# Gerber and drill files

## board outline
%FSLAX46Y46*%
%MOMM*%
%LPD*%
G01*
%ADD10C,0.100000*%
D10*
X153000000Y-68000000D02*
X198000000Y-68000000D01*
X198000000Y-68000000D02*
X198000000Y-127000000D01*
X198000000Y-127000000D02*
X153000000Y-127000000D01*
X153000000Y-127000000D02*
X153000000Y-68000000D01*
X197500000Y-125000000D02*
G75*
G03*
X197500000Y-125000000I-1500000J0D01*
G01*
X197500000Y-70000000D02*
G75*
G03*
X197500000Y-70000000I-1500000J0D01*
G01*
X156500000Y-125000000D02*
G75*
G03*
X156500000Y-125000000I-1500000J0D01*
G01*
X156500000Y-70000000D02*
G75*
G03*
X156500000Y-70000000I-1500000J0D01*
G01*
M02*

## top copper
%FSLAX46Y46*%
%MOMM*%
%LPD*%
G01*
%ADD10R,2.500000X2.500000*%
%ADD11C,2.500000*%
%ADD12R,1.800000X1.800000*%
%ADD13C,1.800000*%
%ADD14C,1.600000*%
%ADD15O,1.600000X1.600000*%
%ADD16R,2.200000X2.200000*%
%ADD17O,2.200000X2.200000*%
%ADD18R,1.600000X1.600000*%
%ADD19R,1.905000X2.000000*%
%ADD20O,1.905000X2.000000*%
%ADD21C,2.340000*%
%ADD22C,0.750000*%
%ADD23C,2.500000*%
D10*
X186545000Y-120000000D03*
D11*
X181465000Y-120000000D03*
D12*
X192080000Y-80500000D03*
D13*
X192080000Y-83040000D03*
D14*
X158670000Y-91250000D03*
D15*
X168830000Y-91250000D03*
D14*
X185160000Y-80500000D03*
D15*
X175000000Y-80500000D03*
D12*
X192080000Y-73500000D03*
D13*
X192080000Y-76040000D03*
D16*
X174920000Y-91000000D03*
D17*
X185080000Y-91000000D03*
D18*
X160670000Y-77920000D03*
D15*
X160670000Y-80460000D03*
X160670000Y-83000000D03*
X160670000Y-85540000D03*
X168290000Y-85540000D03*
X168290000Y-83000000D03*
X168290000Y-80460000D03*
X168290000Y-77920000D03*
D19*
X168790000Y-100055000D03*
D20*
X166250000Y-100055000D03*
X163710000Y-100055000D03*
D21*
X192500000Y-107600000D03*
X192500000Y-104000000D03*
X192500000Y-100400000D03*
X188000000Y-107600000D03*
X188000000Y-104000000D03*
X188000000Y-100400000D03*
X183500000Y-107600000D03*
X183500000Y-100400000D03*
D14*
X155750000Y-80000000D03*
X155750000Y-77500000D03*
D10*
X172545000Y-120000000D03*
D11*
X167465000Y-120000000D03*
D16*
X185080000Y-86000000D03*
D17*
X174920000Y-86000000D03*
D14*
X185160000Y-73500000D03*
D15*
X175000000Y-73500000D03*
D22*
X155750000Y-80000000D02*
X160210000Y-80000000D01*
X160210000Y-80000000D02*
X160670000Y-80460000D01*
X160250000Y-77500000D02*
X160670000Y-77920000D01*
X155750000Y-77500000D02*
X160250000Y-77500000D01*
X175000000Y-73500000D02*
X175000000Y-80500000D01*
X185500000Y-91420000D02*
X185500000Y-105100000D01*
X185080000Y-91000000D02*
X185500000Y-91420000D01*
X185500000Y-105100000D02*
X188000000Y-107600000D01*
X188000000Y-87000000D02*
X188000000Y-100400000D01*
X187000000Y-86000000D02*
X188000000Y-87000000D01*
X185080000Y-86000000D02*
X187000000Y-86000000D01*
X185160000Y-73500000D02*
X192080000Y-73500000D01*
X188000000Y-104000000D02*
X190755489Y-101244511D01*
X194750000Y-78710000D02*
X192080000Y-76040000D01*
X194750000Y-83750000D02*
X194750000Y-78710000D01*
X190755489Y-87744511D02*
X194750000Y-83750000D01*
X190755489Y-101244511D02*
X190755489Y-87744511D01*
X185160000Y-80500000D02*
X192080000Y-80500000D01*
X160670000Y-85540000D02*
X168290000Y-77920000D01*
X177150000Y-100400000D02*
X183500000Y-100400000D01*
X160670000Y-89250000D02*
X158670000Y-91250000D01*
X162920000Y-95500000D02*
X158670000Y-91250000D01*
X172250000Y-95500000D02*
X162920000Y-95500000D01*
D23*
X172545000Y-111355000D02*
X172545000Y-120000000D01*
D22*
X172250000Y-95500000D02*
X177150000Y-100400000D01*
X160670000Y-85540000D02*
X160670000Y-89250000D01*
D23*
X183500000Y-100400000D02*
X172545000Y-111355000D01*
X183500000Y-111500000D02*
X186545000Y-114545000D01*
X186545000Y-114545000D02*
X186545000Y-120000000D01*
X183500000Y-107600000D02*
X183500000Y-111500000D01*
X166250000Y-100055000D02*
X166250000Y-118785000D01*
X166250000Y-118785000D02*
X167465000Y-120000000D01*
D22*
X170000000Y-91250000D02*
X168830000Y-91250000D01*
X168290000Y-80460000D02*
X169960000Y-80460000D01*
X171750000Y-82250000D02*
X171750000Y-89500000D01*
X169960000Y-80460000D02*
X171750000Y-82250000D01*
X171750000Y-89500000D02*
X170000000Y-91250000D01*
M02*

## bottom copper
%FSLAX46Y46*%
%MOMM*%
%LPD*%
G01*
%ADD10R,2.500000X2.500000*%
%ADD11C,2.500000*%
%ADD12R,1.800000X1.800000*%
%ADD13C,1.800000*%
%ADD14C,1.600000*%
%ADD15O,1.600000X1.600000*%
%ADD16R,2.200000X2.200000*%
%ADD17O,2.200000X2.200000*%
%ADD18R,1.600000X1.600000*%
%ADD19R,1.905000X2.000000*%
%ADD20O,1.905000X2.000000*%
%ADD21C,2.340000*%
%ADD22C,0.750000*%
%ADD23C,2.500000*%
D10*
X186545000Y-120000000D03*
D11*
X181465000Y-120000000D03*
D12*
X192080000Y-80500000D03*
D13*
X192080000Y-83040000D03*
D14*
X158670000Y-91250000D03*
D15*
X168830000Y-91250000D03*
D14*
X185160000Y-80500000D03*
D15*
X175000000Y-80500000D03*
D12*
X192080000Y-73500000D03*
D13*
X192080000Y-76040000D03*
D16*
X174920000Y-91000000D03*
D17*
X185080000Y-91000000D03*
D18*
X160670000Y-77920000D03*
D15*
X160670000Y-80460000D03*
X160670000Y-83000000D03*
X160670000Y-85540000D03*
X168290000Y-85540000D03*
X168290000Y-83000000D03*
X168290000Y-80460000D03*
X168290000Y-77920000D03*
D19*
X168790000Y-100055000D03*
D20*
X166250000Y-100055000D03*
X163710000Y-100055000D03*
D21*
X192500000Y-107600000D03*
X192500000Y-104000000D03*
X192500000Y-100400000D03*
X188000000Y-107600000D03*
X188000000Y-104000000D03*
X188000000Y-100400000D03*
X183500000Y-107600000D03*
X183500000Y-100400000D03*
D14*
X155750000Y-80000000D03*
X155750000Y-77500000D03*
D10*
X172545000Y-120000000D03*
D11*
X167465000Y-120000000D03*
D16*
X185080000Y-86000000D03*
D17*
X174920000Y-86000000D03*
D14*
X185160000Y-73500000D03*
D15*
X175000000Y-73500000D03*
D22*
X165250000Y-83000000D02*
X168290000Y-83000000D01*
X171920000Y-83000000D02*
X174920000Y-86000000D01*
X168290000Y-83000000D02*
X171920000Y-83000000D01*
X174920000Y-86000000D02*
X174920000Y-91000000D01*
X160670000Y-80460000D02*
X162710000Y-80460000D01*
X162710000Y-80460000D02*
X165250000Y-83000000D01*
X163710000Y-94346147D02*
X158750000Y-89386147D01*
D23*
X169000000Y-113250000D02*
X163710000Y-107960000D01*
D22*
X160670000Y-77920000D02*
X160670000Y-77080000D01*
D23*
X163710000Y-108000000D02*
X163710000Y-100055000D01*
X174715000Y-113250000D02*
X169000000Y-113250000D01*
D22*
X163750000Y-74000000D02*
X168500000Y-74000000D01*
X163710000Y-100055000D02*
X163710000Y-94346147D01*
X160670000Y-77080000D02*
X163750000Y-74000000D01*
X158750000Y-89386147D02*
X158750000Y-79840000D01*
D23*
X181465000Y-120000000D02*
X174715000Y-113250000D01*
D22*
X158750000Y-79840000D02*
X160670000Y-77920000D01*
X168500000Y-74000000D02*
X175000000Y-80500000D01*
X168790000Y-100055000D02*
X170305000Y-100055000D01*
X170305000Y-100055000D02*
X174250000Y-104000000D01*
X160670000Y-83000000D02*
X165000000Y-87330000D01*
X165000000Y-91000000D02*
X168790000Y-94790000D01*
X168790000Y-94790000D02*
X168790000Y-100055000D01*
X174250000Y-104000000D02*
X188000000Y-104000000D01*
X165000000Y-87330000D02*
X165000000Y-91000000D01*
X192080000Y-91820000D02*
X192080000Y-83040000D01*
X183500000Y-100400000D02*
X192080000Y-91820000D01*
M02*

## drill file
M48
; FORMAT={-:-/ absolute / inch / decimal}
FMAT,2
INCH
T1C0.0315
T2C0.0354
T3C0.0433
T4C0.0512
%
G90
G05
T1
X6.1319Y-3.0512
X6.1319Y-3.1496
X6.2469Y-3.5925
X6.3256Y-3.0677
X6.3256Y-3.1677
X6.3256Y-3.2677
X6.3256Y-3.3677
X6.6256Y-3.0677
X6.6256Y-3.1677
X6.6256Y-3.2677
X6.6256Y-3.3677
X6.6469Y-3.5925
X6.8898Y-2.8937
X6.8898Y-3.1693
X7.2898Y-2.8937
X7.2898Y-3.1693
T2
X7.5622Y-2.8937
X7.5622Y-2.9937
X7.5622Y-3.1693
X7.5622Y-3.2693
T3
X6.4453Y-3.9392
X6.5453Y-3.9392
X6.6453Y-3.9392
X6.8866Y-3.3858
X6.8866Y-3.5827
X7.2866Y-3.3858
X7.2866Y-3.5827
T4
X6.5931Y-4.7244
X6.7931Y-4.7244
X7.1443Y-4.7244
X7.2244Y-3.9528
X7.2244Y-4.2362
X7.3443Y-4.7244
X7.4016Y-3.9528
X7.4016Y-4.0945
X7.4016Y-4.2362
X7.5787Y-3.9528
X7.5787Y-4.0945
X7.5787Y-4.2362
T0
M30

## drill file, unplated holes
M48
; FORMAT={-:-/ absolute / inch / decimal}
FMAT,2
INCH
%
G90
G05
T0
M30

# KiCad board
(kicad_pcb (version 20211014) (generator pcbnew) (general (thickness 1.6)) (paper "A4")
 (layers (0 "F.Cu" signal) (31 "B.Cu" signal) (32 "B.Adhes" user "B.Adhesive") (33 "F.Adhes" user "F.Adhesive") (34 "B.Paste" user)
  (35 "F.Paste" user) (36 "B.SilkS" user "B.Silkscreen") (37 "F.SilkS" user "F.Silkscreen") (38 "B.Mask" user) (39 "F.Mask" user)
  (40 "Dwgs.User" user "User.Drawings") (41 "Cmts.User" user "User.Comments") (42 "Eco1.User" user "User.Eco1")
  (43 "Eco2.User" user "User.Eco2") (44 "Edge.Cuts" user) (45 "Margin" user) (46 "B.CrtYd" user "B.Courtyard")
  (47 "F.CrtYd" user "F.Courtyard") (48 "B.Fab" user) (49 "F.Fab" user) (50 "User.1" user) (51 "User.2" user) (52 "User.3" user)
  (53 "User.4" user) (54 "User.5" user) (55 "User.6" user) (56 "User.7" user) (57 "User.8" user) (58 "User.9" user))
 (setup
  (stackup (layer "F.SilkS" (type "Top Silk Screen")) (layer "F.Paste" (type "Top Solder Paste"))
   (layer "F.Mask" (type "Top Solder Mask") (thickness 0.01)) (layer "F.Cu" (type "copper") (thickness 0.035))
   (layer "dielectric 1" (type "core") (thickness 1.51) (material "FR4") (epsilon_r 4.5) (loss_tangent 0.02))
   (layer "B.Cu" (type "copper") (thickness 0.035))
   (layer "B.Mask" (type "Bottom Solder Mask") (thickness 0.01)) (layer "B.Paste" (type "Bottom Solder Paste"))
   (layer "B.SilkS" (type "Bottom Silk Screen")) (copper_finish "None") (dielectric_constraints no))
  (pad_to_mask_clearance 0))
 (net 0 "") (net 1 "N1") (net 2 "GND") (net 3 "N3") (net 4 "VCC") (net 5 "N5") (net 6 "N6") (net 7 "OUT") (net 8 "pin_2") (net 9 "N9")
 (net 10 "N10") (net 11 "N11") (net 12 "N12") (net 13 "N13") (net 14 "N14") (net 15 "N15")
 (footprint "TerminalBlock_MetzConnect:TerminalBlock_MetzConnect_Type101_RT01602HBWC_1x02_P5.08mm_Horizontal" (layer "F.Cu")
  (at 186.545 120 180)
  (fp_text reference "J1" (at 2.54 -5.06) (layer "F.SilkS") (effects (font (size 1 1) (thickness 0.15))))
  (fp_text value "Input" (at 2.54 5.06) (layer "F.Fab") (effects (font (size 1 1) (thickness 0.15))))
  (pad "1" thru_hole rect (at 0 0 180) (size 2.5 2.5) (drill 1.3) (layers *.Cu *.Mask) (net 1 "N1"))
  (pad "2" thru_hole circle (at 5.08 0 180) (size 2.5 2.5) (drill 1.3) (layers *.Cu *.Mask) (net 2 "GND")))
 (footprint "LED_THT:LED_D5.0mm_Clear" (layer "F.Cu") (at 192.08 80.5 -90)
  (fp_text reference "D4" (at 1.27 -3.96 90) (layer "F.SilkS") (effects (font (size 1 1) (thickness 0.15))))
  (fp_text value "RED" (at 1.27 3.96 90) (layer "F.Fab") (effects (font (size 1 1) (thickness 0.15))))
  (pad "1" thru_hole rect (at 0 0 270) (size 1.8 1.8) (drill 0.9) (layers *.Cu *.Mask) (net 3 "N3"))
  (pad "2" thru_hole circle (at 2.54 0 270) (size 1.8 1.8) (drill 0.9) (layers *.Cu *.Mask) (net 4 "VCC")))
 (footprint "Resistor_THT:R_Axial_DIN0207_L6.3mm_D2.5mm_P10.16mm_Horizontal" (layer "F.Cu") (at 158.67 91.25)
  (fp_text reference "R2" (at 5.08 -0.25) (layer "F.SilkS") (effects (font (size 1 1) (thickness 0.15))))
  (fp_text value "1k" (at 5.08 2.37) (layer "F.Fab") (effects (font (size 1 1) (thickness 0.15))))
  (pad "1" thru_hole circle (at 0 0) (size 1.6 1.6) (drill 0.8) (layers *.Cu *.Mask) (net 4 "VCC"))
  (pad "2" thru_hole oval (at 10.16 0) (size 1.6 1.6) (drill 0.8) (layers *.Cu *.Mask) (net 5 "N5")))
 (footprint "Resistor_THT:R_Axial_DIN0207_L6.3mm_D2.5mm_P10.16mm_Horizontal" (layer "F.Cu") (at 185.16 80.5 180)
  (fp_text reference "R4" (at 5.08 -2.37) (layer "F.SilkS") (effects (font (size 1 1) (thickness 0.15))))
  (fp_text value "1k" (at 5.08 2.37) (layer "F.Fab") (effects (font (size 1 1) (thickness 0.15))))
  (pad "1" thru_hole circle (at 0 0 180) (size 1.6 1.6) (drill 0.8) (layers *.Cu *.Mask) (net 3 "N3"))
  (pad "2" thru_hole oval (at 10.16 0 180) (size 1.6 1.6) (drill 0.8) (layers *.Cu *.Mask) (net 2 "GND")))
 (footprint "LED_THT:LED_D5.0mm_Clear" (layer "F.Cu") (at 192.08 73.5 -90)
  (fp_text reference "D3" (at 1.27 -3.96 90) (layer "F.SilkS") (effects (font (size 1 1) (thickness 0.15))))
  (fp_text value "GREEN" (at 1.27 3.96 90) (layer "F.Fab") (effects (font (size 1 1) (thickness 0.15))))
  (pad "1" thru_hole rect (at 0 0 270) (size 1.8 1.8) (drill 0.9) (layers *.Cu *.Mask) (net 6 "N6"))
  (pad "2" thru_hole circle (at 2.54 0 270) (size 1.8 1.8) (drill 0.9) (layers *.Cu *.Mask) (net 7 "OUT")))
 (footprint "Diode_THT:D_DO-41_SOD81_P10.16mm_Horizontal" (layer "F.Cu") (at 174.92 91)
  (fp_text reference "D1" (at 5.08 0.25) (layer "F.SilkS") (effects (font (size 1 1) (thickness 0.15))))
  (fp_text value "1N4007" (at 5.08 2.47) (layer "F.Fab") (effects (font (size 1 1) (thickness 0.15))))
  (pad "1" thru_hole rect (at 0 0) (size 2.2 2.2) (drill 1.1) (layers *.Cu *.Mask) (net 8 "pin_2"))
  (pad "2" thru_hole oval (at 10.16 0) (size 2.2 2.2) (drill 1.1) (layers *.Cu *.Mask) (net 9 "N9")))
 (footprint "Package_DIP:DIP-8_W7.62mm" (layer "F.Cu") (at 160.67 77.92)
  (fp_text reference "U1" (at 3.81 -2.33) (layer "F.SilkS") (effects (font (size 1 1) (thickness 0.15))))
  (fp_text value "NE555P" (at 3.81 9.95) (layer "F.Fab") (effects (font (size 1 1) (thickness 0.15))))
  (pad "1" thru_hole rect (at 0 0) (size 1.6 1.6) (drill 0.8) (layers *.Cu *.Mask) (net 2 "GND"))
  (pad "2" thru_hole oval (at 0 2.54) (size 1.6 1.6) (drill 0.8) (layers *.Cu *.Mask) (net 8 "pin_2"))
  (pad "3" thru_hole oval (at 0 5.08) (size 1.6 1.6) (drill 0.8) (layers *.Cu *.Mask) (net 7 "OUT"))
  (pad "4" thru_hole oval (at 0 7.62) (size 1.6 1.6) (drill 0.8) (layers *.Cu *.Mask) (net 4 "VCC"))
  (pad "5" thru_hole oval (at 7.62 7.62) (size 1.6 1.6) (drill 0.8) (layers *.Cu *.Mask) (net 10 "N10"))
  (pad "6" thru_hole oval (at 7.62 5.08) (size 1.6 1.6) (drill 0.8) (layers *.Cu *.Mask) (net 8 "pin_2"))
  (pad "7" thru_hole oval (at 7.62 2.54) (size 1.6 1.6) (drill 0.8) (layers *.Cu *.Mask) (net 5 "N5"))
  (pad "8" thru_hole oval (at 7.62 0) (size 1.6 1.6) (drill 0.8) (layers *.Cu *.Mask) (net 4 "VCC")))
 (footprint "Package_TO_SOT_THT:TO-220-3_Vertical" (layer "F.Cu") (at 168.79 100.055 180)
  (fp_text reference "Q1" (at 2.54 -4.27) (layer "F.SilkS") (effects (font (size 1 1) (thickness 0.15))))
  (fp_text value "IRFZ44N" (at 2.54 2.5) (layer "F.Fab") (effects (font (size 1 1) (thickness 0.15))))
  (pad "1" thru_hole rect (at 0 0 180) (size 1.905 2) (drill 1.1) (layers *.Cu *.Mask) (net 7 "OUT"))
  (pad "2" thru_hole oval (at 2.54 0 180) (size 1.905 2) (drill 1.1) (layers *.Cu *.Mask) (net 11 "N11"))
  (pad "3" thru_hole oval (at 5.08 0 180) (size 1.905 2) (drill 1.1) (layers *.Cu *.Mask) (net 2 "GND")))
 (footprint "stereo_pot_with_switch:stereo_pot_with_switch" (layer "F.Cu") (at 186.5 104)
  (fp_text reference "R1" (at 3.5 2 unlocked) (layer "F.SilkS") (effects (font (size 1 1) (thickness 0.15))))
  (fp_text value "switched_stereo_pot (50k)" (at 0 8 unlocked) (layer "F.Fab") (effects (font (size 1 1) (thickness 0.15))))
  (pad "1" thru_hole circle (at 6 3.6) (size 2.34 2.34) (drill 1.3) (layers *.Cu *.Mask) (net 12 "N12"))
  (pad "2" thru_hole circle (at 6 0) (size 2.34 2.34) (drill 1.3) (layers *.Cu *.Mask) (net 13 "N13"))
  (pad "3" thru_hole circle (at 6 -3.6) (size 2.34 2.34) (drill 1.3) (layers *.Cu *.Mask) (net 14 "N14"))
  (pad "4" thru_hole circle (at 1.5 3.6) (size 2.34 2.34) (drill 1.3) (layers *.Cu *.Mask) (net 9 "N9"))
  (pad "5" thru_hole circle (at 1.5 0) (size 2.34 2.34) (drill 1.3) (layers *.Cu *.Mask) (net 7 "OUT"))
  (pad "6" thru_hole circle (at 1.5 -3.6) (size 2.34 2.34) (drill 1.3) (layers *.Cu *.Mask) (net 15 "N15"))
  (pad "7" thru_hole circle (at -3 3.6) (size 2.34 2.34) (drill 1.3) (layers *.Cu *.Mask) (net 1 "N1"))
  (pad "8" thru_hole circle (at -3 -3.6) (size 2.34 2.34) (drill 1.3) (layers *.Cu *.Mask) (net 4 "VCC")))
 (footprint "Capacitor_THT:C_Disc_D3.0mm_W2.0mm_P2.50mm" (layer "F.Cu") (at 155.75 80 90)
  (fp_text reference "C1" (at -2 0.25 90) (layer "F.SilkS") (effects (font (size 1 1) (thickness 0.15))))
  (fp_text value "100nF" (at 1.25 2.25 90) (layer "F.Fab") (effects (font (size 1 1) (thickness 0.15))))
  (pad "1" thru_hole circle (at 0 0 90) (size 1.6 1.6) (drill 0.8) (layers *.Cu *.Mask) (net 8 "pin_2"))
  (pad "2" thru_hole circle (at 2.5 0 90) (size 1.6 1.6) (drill 0.8) (layers *.Cu *.Mask) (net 2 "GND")))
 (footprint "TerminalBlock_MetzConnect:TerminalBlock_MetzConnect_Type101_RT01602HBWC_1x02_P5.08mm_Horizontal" (layer "F.Cu")
  (at 172.545 120 180)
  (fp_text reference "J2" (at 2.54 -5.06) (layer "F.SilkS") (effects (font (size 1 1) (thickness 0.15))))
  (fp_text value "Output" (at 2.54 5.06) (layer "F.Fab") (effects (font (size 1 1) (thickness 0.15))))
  (pad "1" thru_hole rect (at 0 0 180) (size 2.5 2.5) (drill 1.3) (layers *.Cu *.Mask) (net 4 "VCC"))
  (pad "2" thru_hole circle (at 5.08 0 180) (size 2.5 2.5) (drill 1.3) (layers *.Cu *.Mask) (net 11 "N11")))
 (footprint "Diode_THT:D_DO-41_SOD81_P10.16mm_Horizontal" (layer "F.Cu") (at 185.08 86 180)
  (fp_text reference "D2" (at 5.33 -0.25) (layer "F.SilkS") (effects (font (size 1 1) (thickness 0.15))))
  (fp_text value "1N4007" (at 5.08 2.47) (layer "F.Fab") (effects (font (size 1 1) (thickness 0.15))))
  (pad "1" thru_hole rect (at 0 0 180) (size 2.2 2.2) (drill 1.1) (layers *.Cu *.Mask) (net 15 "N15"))
  (pad "2" thru_hole oval (at 10.16 0 180) (size 2.2 2.2) (drill 1.1) (layers *.Cu *.Mask) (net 8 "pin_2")))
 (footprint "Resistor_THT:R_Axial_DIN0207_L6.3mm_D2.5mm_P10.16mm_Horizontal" (layer "F.Cu") (at 185.16 73.5 180)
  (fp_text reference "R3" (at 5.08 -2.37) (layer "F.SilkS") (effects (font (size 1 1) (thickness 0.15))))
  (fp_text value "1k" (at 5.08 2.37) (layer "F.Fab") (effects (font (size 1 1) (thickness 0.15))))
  (pad "1" thru_hole circle (at 0 0 180) (size 1.6 1.6) (drill 0.8) (layers *.Cu *.Mask) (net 6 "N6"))
  (pad "2" thru_hole oval (at 10.16 0 180) (size 1.6 1.6) (drill 0.8) (layers *.Cu *.Mask) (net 2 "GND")))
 (gr_rect (start 153 68) (end 198 127) (layer "Edge.Cuts") (width 0.1) (fill none))
 (gr_circle (center 196 125) (end 197.5 125) (layer "Edge.Cuts") (width 0.1) (fill none))
 (gr_circle (center 196 70) (end 197.5 70) (layer "Edge.Cuts") (width 0.1) (fill none))
 (gr_circle (center 155 125) (end 156.5 125) (layer "Edge.Cuts") (width 0.1) (fill none))
 (gr_circle (center 155 70) (end 156.5 70) (layer "Edge.Cuts") (width 0.1) (fill none))
 (segment (start 155.75 80) (end 160.21 80) (width 0.75) (layer "F.Cu") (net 8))
 (segment (start 160.21 80) (end 160.67 80.46) (width 0.75) (layer "F.Cu") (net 8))
 (segment (start 165.25 83) (end 168.29 83) (width 0.75) (layer "B.Cu") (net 8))
 (segment (start 171.92 83) (end 174.92 86) (width 0.75) (layer "B.Cu") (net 8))
 (segment (start 168.29 83) (end 171.92 83) (width 0.75) (layer "B.Cu") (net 8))
 (segment (start 174.92 86) (end 174.92 91) (width 0.75) (layer "B.Cu") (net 8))
 (segment (start 160.67 80.46) (end 162.71 80.46) (width 0.75) (layer "B.Cu") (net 8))
 (segment (start 162.71 80.46) (end 165.25 83) (width 0.75) (layer "B.Cu") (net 8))
 (segment (start 160.25 77.5) (end 160.67 77.92) (width 0.75) (layer "F.Cu") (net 2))
 (segment (start 155.75 77.5) (end 160.25 77.5) (width 0.75) (layer "F.Cu") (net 2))
 (segment (start 175 73.5) (end 175 80.5) (width 0.75) (layer "F.Cu") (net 2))
 (segment (start 163.71 94.346147) (end 158.75 89.386147) (width 0.75) (layer "B.Cu") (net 2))
 (segment (start 169 113.25) (end 163.71 107.96) (width 2.5) (layer "B.Cu") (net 2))
 (segment (start 160.67 77.92) (end 160.67 77.08) (width 0.75) (layer "B.Cu") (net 2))
 (segment (start 163.71 108) (end 163.71 100.055) (width 2.5) (layer "B.Cu") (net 2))
 (segment (start 174.715 113.25) (end 169 113.25) (width 2.5) (layer "B.Cu") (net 2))
 (segment (start 163.75 74) (end 168.5 74) (width 0.75) (layer "B.Cu") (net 2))
 (segment (start 163.71 100.055) (end 163.71 94.346147) (width 0.75) (layer "B.Cu") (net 2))
 (segment (start 160.67 77.08) (end 163.75 74) (width 0.75) (layer "B.Cu") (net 2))
 (segment (start 158.75 89.386147) (end 158.75 79.84) (width 0.75) (layer "B.Cu") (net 2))
 (segment (start 181.465 120) (end 174.715 113.25) (width 2.5) (layer "B.Cu") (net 2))
 (segment (start 158.75 79.84) (end 160.67 77.92) (width 0.75) (layer "B.Cu") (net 2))
 (segment (start 168.5 74) (end 175 80.5) (width 0.75) (layer "B.Cu") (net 2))
 (segment (start 185.5 91.42) (end 185.5 105.1) (width 0.75) (layer "F.Cu") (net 9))
 (segment (start 185.08 91) (end 185.5 91.42) (width 0.75) (layer "F.Cu") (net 9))
 (segment (start 185.5 105.1) (end 188 107.6) (width 0.75) (layer "F.Cu") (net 9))
 (segment (start 188 87) (end 188 100.4) (width 0.75) (layer "F.Cu") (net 15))
 (segment (start 187 86) (end 188 87) (width 0.75) (layer "F.Cu") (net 15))
 (segment (start 185.08 86) (end 187 86) (width 0.75) (layer "F.Cu") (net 15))
 (segment (start 185.16 73.5) (end 192.08 73.5) (width 0.75) (layer "F.Cu") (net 6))
 (segment (start 188 104) (end 190.755489 101.244511) (width 0.75) (layer "F.Cu") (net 7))
 (segment (start 194.75 78.71) (end 192.08 76.04) (width 0.75) (layer "F.Cu") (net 7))
 (segment (start 194.75 83.75) (end 194.75 78.71) (width 0.75) (layer "F.Cu") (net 7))
 (segment (start 190.755489 87.744511) (end 194.75 83.75) (width 0.75) (layer "F.Cu") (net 7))
 (segment (start 190.755489 101.244511) (end 190.755489 87.744511) (width 0.75) (layer "F.Cu") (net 7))
 (segment (start 168.79 100.055) (end 170.305 100.055) (width 0.75) (layer "B.Cu") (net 7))
 (segment (start 170.305 100.055) (end 174.25 104) (width 0.75) (layer "B.Cu") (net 7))
 (segment (start 160.67 83) (end 165 87.33) (width 0.75) (layer "B.Cu") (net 7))
 (segment (start 165 91) (end 168.79 94.79) (width 0.75) (layer "B.Cu") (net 7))
 (segment (start 168.79 94.79) (end 168.79 100.055) (width 0.75) (layer "B.Cu") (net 7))
 (segment (start 174.25 104) (end 188 104) (width 0.75) (layer "B.Cu") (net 7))
 (segment (start 165 87.33) (end 165 91) (width 0.75) (layer "B.Cu") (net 7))
 (segment (start 185.16 80.5) (end 192.08 80.5) (width 0.75) (layer "F.Cu") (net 3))
 (segment (start 160.67 85.54) (end 168.29 77.92) (width 0.75) (layer "F.Cu") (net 4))
 (segment (start 177.15 100.4) (end 183.5 100.4) (width 0.75) (layer "F.Cu") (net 4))
 (segment (start 160.67 89.25) (end 158.67 91.25) (width 0.75) (layer "F.Cu") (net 4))
 (segment (start 162.92 95.5) (end 158.67 91.25) (width 0.75) (layer "F.Cu") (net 4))
 (segment (start 172.25 95.5) (end 162.92 95.5) (width 0.75) (layer "F.Cu") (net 4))
 (segment (start 172.545 111.355) (end 172.545 120) (width 2.5) (layer "F.Cu") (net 4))
 (segment (start 172.25 95.5) (end 177.15 100.4) (width 0.75) (layer "F.Cu") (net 4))
 (segment (start 160.67 85.54) (end 160.67 89.25) (width 0.75) (layer "F.Cu") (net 4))
 (segment (start 183.5 100.4) (end 172.545 111.355) (width 2.5) (layer "F.Cu") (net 4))
 (segment (start 192.08 91.82) (end 192.08 83.04) (width 0.75) (layer "B.Cu") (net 4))
 (segment (start 183.5 100.4) (end 192.08 91.82) (width 0.75) (layer "B.Cu") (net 4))
 (segment (start 183.5 111.5) (end 186.545 114.545) (width 2.5) (layer "F.Cu") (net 1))
 (segment (start 186.545 114.545) (end 186.545 120) (width 2.5) (layer "F.Cu") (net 1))
 (segment (start 183.5 107.6) (end 183.5 111.5) (width 2.5) (layer "F.Cu") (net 1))
 (segment (start 166.25 100.055) (end 166.25 118.785) (width 2.5) (layer "F.Cu") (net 11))
 (segment (start 166.25 118.785) (end 167.465 120) (width 2.5) (layer "F.Cu") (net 11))
 (segment (start 170 91.25) (end 168.83 91.25) (width 0.75) (layer "F.Cu") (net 5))
 (segment (start 168.29 80.46) (end 169.96 80.46) (width 0.75) (layer "F.Cu") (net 5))
 (segment (start 171.75 82.25) (end 171.75 89.5) (width 0.75) (layer "F.Cu") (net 5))
 (segment (start 169.96 80.46) (end 171.75 82.25) (width 0.75) (layer "F.Cu") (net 5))
 (segment (start 171.75 89.5) (end 170 91.25) (width 0.75) (layer "F.Cu") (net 5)))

